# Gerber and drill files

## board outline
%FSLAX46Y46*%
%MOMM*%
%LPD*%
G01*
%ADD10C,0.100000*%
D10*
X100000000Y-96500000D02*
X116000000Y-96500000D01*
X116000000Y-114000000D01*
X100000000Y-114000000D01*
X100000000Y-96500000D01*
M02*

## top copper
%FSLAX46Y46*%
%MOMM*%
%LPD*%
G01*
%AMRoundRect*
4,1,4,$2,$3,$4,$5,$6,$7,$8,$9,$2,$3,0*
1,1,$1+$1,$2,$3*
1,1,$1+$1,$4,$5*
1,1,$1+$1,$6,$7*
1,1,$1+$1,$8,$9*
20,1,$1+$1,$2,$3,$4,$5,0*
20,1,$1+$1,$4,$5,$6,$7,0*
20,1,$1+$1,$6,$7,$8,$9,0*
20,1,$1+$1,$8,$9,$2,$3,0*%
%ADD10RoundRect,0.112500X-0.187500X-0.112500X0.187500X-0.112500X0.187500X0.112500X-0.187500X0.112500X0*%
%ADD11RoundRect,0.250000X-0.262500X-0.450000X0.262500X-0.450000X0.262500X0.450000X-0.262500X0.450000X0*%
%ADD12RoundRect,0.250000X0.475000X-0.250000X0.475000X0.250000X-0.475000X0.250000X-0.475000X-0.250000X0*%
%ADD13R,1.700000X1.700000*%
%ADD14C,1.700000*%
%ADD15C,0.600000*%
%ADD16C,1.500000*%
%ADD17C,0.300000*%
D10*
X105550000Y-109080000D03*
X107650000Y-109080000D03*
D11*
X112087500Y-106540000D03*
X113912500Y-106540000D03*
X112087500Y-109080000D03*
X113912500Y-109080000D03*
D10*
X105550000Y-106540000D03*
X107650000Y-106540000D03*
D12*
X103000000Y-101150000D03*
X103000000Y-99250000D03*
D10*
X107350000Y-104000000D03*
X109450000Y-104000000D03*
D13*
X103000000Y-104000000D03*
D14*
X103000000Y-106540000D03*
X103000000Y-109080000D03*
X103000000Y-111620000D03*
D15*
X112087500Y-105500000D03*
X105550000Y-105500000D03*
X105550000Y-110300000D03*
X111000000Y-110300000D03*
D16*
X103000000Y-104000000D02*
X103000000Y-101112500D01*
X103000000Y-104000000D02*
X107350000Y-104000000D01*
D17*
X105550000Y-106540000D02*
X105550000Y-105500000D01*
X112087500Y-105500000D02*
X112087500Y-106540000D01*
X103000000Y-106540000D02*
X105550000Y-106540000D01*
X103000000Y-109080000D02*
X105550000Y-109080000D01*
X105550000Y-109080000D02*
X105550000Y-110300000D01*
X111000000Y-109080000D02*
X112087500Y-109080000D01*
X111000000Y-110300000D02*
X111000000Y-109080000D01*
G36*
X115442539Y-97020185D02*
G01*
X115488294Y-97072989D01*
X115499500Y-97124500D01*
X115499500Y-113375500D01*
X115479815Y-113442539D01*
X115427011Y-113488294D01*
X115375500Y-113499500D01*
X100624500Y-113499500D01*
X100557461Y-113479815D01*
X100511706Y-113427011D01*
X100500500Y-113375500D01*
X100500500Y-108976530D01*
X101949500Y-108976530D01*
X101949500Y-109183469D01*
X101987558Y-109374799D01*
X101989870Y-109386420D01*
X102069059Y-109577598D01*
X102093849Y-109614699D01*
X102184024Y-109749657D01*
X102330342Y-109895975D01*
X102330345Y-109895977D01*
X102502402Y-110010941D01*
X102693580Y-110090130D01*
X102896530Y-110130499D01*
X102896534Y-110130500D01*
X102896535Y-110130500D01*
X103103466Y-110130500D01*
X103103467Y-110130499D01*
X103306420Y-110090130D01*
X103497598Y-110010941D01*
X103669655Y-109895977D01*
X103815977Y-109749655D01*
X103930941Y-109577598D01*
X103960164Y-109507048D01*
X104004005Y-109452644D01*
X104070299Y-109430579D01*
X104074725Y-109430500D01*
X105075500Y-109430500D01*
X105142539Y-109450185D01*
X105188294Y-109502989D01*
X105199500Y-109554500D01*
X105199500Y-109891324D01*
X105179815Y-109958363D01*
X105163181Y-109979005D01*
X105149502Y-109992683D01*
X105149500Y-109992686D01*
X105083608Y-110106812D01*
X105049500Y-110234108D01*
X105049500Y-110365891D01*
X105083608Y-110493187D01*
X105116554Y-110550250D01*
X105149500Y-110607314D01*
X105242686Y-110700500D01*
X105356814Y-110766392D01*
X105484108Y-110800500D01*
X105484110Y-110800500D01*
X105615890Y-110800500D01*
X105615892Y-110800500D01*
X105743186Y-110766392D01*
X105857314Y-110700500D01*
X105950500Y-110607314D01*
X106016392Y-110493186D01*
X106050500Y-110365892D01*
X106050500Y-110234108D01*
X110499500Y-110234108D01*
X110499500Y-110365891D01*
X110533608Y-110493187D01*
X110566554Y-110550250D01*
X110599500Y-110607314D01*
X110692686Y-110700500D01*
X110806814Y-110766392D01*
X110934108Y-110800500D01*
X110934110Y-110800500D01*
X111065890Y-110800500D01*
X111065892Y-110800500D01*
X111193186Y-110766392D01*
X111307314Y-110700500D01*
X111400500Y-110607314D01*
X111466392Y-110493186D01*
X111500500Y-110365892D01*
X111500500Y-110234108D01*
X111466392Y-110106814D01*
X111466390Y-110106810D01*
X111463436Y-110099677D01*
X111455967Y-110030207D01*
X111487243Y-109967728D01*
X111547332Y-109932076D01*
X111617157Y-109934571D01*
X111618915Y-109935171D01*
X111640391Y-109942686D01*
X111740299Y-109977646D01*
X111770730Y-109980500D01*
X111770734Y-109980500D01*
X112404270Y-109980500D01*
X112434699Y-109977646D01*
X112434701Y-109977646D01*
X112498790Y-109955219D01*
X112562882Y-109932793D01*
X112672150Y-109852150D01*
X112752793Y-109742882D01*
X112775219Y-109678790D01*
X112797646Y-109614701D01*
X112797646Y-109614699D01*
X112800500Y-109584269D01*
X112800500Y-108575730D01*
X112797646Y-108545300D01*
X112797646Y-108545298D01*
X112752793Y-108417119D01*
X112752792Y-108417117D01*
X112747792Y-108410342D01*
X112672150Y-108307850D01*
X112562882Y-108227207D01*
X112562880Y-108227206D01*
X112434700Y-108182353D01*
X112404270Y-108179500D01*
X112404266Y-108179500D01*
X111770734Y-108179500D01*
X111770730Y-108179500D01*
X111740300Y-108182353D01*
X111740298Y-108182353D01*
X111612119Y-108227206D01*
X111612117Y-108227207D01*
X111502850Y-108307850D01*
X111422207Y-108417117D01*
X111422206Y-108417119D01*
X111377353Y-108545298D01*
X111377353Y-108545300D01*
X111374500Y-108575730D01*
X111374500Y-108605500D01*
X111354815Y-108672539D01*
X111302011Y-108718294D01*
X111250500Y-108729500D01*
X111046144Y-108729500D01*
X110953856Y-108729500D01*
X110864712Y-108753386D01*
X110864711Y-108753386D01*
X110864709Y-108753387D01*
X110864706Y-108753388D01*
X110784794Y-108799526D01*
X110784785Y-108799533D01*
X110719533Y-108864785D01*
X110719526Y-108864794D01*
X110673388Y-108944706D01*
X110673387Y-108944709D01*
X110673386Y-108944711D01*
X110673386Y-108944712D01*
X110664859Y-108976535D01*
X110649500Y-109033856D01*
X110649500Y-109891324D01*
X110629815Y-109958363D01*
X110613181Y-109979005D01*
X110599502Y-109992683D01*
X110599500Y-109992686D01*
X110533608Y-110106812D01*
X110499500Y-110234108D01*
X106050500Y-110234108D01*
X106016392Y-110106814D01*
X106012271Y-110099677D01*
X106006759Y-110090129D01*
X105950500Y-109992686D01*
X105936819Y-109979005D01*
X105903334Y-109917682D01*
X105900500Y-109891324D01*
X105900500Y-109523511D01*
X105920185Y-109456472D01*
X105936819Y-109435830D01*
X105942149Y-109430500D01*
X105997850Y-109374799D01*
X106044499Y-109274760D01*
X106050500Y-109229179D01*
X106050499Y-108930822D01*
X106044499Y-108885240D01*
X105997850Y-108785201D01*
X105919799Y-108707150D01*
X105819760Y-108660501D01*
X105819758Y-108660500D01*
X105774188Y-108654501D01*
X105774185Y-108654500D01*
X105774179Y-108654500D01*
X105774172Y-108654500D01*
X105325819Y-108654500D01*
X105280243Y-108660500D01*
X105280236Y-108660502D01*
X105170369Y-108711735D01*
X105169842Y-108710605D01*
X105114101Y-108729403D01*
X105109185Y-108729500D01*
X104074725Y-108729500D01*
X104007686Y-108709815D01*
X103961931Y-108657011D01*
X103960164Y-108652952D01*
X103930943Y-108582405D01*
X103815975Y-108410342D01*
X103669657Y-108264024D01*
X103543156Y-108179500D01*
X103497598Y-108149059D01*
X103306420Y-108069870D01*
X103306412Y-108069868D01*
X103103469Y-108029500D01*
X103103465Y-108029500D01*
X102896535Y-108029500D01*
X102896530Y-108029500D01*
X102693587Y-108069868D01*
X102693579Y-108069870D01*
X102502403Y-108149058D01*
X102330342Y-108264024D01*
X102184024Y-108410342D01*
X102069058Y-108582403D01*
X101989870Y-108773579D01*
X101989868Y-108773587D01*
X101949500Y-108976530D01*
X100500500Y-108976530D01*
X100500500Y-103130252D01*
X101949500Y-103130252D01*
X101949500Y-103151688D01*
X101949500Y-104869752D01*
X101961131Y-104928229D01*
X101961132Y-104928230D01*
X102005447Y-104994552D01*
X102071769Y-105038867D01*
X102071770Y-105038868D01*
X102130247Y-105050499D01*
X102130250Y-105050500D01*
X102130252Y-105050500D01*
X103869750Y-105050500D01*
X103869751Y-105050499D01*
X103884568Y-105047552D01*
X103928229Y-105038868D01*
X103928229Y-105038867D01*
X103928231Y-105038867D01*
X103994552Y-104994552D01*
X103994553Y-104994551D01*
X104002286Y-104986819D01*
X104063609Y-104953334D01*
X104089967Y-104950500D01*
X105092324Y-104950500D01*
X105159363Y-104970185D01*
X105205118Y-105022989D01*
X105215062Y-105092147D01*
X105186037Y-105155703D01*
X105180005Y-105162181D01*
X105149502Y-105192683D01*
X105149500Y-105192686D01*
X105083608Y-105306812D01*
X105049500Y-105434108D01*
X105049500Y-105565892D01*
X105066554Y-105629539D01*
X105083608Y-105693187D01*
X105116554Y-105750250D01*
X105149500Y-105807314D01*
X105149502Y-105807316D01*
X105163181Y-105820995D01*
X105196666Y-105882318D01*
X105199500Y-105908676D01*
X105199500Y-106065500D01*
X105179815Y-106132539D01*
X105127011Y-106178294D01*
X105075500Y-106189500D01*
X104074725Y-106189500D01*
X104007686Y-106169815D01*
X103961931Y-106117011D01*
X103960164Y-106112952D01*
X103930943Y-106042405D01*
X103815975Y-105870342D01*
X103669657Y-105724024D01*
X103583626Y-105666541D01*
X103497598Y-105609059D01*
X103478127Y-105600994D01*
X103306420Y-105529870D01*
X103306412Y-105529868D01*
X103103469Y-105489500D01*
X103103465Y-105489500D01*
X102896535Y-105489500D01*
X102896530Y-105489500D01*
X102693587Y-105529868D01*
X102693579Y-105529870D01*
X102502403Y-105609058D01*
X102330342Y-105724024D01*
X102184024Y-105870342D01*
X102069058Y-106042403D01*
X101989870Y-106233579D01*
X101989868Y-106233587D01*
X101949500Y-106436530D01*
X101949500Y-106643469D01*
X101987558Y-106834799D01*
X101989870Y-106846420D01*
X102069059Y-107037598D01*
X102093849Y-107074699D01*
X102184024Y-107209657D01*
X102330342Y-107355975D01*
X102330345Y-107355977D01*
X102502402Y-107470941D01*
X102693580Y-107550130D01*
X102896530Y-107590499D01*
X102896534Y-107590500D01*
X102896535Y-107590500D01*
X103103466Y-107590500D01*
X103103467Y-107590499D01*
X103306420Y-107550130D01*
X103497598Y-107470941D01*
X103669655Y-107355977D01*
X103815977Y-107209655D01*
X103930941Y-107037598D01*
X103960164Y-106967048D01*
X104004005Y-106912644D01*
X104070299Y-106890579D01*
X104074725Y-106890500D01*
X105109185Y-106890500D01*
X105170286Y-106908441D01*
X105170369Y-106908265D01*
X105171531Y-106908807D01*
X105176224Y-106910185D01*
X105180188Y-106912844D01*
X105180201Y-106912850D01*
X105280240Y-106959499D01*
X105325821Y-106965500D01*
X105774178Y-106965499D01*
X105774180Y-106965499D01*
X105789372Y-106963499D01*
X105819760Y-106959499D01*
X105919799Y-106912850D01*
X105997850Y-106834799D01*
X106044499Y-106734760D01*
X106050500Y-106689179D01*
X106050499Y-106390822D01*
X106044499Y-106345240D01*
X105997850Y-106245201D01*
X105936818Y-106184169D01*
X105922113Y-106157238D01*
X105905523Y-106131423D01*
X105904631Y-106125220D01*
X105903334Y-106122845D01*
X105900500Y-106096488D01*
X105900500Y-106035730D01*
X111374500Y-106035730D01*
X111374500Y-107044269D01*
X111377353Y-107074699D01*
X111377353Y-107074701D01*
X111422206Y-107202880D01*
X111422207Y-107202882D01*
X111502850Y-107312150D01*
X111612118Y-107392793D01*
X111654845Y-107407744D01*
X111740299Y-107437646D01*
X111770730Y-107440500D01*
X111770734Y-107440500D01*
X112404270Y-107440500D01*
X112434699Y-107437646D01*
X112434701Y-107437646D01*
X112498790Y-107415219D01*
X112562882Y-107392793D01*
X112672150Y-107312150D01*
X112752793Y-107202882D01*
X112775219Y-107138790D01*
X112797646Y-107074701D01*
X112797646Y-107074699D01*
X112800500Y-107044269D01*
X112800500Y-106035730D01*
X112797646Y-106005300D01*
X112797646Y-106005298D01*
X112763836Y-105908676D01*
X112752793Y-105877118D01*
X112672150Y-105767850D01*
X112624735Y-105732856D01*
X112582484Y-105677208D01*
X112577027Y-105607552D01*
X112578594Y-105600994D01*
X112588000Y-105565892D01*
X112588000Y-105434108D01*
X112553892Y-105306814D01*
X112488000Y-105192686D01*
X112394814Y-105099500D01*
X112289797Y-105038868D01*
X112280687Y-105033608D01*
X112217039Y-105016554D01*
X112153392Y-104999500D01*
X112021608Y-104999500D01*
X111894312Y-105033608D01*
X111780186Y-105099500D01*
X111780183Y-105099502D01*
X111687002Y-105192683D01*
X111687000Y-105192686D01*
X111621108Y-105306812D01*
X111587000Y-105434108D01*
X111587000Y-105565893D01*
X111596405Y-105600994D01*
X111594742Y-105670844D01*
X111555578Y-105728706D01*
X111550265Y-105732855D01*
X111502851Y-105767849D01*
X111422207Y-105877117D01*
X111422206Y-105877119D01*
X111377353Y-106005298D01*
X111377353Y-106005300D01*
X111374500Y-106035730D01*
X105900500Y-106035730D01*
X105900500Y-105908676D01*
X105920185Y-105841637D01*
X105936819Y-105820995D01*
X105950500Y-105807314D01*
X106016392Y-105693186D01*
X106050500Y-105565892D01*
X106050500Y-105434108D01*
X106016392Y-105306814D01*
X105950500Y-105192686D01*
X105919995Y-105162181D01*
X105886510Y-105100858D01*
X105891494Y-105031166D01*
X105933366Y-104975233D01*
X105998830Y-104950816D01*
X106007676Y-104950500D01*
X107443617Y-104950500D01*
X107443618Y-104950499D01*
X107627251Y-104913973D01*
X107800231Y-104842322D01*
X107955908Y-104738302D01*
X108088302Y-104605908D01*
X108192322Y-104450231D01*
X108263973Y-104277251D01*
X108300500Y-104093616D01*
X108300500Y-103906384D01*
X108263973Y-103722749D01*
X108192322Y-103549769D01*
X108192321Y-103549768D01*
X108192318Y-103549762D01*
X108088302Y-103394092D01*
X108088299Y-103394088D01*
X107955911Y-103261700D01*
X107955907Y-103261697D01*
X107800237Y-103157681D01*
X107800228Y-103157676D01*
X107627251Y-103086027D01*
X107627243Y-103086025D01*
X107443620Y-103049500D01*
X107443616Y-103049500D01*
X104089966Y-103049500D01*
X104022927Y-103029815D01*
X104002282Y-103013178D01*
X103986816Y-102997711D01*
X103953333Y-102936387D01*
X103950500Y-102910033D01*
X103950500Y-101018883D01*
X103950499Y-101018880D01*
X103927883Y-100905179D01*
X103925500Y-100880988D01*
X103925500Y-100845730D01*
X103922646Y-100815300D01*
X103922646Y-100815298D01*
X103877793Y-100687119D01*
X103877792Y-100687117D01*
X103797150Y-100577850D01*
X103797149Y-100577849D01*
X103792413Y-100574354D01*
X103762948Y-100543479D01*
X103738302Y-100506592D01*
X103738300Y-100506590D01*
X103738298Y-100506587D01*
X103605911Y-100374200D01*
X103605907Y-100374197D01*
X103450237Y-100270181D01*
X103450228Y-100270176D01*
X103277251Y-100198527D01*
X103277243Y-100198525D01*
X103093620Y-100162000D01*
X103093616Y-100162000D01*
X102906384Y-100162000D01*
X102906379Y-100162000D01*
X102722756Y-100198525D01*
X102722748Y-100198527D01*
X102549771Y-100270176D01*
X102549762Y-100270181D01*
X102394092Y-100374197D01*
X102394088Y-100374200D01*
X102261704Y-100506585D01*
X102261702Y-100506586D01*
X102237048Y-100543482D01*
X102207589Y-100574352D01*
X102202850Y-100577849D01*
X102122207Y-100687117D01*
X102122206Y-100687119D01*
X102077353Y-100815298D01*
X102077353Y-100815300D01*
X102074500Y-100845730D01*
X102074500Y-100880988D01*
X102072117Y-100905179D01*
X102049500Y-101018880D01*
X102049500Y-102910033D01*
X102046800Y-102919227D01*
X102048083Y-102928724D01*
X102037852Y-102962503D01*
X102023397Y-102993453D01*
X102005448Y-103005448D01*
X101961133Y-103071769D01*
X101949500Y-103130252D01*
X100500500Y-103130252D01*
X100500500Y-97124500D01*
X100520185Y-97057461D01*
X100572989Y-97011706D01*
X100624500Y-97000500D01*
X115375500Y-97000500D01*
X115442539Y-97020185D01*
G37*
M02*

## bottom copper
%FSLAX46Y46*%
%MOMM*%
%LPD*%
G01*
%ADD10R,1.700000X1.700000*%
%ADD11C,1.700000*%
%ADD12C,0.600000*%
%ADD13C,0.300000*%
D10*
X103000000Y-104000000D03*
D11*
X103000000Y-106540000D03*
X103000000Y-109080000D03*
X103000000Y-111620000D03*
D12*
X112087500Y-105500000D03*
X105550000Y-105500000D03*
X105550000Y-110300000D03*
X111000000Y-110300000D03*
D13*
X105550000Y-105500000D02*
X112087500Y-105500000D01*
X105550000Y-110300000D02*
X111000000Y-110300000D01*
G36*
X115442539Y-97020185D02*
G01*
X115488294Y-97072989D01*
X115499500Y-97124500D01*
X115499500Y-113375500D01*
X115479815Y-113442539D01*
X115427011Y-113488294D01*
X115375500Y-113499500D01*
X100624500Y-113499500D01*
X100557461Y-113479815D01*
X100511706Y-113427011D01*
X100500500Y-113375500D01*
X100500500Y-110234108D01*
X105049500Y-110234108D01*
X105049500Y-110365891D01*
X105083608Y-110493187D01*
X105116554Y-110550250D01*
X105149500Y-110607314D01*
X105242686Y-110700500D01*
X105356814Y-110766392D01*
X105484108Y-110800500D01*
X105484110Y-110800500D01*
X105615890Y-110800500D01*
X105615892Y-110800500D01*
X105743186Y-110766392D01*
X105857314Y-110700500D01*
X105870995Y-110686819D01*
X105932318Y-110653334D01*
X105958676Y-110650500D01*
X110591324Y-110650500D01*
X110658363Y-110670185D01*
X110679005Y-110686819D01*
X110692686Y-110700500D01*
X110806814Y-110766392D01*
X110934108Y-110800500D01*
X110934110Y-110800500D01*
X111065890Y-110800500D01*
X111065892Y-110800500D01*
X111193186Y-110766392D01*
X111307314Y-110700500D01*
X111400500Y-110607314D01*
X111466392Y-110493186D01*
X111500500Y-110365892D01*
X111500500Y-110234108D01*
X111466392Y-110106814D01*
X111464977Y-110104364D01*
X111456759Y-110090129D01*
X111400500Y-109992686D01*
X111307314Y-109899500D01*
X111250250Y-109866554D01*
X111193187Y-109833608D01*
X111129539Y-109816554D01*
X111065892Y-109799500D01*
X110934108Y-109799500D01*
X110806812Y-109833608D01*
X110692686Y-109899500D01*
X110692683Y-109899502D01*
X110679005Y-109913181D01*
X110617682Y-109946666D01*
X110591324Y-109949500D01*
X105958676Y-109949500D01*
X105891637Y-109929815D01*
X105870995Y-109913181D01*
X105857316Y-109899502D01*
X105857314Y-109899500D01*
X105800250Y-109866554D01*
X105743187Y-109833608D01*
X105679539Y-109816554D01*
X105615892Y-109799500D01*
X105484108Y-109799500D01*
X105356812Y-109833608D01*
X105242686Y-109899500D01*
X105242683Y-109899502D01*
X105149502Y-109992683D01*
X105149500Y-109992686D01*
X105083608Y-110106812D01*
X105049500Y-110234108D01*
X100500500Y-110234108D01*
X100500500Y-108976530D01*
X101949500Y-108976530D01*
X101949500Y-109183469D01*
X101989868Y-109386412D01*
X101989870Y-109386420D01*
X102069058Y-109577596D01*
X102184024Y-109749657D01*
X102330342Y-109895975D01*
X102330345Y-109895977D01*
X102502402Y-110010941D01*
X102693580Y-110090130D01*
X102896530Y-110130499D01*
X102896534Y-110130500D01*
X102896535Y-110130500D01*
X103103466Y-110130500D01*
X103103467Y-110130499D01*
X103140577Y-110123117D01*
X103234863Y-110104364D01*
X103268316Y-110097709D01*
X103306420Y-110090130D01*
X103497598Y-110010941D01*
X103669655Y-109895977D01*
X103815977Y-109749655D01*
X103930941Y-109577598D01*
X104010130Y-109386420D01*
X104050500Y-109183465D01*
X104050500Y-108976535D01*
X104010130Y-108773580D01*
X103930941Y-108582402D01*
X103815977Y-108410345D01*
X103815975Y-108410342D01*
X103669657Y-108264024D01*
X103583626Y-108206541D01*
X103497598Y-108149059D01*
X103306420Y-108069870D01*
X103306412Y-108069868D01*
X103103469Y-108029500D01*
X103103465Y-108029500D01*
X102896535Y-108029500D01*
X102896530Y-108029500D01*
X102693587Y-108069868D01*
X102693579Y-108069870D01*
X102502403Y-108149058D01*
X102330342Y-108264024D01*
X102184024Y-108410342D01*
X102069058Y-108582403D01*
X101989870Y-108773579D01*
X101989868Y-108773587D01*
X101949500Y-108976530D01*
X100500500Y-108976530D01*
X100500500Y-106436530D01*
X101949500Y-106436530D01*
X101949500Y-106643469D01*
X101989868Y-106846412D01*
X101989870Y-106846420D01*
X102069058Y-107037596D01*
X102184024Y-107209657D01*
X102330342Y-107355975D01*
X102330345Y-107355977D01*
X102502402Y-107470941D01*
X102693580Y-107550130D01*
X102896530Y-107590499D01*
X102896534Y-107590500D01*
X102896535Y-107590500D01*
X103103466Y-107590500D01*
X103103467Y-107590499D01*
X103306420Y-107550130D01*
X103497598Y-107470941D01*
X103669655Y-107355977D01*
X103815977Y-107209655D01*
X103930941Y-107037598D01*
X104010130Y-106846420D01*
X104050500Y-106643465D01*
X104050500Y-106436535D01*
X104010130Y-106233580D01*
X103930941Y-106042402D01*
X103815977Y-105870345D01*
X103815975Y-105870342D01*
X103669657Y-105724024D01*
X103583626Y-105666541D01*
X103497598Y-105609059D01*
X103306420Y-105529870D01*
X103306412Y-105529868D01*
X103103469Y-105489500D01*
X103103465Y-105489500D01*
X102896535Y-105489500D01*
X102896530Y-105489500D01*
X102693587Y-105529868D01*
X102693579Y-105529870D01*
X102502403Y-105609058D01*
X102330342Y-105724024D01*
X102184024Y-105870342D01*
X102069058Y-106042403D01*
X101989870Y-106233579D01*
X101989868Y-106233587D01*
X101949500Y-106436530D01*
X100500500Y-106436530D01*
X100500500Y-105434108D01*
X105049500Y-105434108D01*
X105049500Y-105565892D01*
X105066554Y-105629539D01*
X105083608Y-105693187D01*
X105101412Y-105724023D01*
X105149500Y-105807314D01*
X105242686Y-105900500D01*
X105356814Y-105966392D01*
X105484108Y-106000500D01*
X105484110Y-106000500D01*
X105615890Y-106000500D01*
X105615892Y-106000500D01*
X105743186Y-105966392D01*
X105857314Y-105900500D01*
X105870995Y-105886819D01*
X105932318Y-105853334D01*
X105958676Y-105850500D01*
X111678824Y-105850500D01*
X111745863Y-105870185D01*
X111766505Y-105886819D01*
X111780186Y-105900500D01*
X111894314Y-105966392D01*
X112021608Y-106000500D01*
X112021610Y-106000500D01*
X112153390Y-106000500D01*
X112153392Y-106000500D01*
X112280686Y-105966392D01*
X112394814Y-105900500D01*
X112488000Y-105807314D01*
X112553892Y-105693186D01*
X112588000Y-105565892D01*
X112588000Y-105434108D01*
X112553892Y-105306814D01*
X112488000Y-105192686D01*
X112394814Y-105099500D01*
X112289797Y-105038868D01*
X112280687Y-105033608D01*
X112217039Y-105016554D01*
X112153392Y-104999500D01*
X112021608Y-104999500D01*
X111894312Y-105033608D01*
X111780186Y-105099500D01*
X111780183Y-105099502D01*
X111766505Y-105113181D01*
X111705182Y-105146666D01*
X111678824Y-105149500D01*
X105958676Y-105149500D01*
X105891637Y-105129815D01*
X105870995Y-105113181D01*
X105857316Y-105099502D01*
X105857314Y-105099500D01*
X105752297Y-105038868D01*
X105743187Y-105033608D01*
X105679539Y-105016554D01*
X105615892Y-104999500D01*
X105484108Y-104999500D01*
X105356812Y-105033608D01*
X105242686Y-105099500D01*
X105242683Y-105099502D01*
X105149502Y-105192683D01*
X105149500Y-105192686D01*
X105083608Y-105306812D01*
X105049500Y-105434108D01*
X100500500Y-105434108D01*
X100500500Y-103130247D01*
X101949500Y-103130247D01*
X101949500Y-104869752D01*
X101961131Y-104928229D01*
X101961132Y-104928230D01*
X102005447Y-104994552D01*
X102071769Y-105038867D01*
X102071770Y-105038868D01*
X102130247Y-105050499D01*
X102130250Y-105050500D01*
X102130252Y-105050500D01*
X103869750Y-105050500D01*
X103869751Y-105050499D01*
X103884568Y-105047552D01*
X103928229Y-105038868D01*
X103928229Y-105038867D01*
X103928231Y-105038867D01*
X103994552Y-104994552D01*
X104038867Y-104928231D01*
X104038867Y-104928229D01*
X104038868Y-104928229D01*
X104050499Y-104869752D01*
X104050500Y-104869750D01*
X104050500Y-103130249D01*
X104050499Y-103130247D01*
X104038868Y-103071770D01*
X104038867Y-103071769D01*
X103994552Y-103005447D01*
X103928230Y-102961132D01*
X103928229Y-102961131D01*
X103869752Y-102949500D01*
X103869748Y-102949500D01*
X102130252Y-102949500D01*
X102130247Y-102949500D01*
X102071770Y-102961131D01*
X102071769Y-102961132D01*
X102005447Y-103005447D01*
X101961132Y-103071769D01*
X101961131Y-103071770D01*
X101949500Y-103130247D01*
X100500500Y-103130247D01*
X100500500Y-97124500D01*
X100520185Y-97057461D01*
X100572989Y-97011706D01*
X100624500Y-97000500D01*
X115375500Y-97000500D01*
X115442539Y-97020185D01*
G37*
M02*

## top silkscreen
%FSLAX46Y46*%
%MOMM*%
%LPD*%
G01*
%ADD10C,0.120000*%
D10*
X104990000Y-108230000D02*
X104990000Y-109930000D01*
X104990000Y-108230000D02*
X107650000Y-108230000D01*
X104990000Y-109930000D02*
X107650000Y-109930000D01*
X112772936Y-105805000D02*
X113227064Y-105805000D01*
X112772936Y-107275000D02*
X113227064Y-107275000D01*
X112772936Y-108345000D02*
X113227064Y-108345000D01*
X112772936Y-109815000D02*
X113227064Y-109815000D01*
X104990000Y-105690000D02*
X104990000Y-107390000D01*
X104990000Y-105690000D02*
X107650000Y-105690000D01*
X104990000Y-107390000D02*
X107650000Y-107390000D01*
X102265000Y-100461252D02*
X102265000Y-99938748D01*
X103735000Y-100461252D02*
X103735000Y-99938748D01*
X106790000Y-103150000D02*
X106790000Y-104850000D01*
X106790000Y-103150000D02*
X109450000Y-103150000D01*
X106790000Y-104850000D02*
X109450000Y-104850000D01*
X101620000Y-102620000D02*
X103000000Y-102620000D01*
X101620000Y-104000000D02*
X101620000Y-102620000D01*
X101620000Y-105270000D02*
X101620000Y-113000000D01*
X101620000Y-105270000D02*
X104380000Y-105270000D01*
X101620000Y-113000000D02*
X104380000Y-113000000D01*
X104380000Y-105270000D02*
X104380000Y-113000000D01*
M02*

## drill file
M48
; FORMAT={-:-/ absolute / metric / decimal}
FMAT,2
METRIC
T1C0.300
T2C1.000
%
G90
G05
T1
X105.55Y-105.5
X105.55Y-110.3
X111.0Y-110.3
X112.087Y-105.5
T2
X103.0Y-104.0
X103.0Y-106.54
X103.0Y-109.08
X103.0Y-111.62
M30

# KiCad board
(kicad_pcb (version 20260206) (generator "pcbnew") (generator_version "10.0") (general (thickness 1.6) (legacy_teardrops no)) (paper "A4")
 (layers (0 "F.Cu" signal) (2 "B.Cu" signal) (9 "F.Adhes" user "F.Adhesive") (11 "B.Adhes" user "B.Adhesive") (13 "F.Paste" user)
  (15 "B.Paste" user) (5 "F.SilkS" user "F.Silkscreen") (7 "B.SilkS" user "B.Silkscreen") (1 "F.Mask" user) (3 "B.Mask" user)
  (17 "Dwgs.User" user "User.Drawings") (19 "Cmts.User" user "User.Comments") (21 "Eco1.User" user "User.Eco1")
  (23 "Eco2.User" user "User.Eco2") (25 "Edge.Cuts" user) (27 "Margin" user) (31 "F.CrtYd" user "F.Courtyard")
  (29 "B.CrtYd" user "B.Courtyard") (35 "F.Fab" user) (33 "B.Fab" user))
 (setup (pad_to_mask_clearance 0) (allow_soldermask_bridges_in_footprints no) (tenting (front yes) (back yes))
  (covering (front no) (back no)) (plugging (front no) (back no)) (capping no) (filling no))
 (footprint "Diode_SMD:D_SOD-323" (layer "F.Cu") (at 106.6 109.08)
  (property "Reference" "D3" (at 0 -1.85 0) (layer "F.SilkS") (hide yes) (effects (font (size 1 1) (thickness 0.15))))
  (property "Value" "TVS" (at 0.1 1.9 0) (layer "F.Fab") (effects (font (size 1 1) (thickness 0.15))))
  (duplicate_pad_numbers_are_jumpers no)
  (fp_line (start -1.61 -0.85) (end -1.61 0.85) (stroke (width 0.12) (type solid)) (layer "F.SilkS"))
  (fp_line (start -1.61 -0.85) (end 1.05 -0.85) (stroke (width 0.12) (type solid)) (layer "F.SilkS"))
  (fp_line (start -1.61 0.85) (end 1.05 0.85) (stroke (width 0.12) (type solid)) (layer "F.SilkS"))
  (pad "1" smd roundrect (at -1.05 0) (size 0.6 0.45) (layers "F.Cu" "F.Mask" "F.Paste") (roundrect_rratio 0.25) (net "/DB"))
  (pad "2" smd roundrect (at 1.05 0) (size 0.6 0.45) (layers "F.Cu" "F.Mask" "F.Paste") (roundrect_rratio 0.25) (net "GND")))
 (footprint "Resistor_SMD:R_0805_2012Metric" (layer "F.Cu") (at 113 106.54)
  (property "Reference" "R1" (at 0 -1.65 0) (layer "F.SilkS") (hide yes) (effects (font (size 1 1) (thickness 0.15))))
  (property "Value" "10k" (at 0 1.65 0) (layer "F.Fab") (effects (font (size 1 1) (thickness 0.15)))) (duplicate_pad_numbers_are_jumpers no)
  (fp_line (start -0.227064 -0.735) (end 0.227064 -0.735) (stroke (width 0.12) (type solid)) (layer "F.SilkS"))
  (fp_line (start -0.227064 0.735) (end 0.227064 0.735) (stroke (width 0.12) (type solid)) (layer "F.SilkS"))
  (pad "1" smd roundrect (at -0.9125 0) (size 1.025 1.4) (layers "F.Cu" "F.Mask" "F.Paste") (roundrect_rratio 0.243902) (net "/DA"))
  (pad "2" smd roundrect (at 0.9125 0) (size 1.025 1.4) (layers "F.Cu" "F.Mask" "F.Paste") (roundrect_rratio 0.243902) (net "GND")))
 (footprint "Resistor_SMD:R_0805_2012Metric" (layer "F.Cu") (at 113 109.08)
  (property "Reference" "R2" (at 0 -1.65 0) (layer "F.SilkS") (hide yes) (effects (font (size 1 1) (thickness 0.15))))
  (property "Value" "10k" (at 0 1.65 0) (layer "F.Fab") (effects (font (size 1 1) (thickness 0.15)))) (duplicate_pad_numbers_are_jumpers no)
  (fp_line (start -0.227064 -0.735) (end 0.227064 -0.735) (stroke (width 0.12) (type solid)) (layer "F.SilkS"))
  (fp_line (start -0.227064 0.735) (end 0.227064 0.735) (stroke (width 0.12) (type solid)) (layer "F.SilkS"))
  (pad "1" smd roundrect (at -0.9125 0) (size 1.025 1.4) (layers "F.Cu" "F.Mask" "F.Paste") (roundrect_rratio 0.243902) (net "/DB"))
  (pad "2" smd roundrect (at 0.9125 0) (size 1.025 1.4) (layers "F.Cu" "F.Mask" "F.Paste") (roundrect_rratio 0.243902) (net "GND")))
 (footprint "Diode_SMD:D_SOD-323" (layer "F.Cu") (at 106.6 106.54)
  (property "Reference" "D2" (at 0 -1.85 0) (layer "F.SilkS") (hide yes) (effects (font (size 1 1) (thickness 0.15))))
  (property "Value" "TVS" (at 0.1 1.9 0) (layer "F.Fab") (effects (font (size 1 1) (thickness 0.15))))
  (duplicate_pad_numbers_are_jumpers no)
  (fp_line (start -1.61 -0.85) (end -1.61 0.85) (stroke (width 0.12) (type solid)) (layer "F.SilkS"))
  (fp_line (start -1.61 -0.85) (end 1.05 -0.85) (stroke (width 0.12) (type solid)) (layer "F.SilkS"))
  (fp_line (start -1.61 0.85) (end 1.05 0.85) (stroke (width 0.12) (type solid)) (layer "F.SilkS"))
  (pad "1" smd roundrect (at -1.05 0) (size 0.6 0.45) (layers "F.Cu" "F.Mask" "F.Paste") (roundrect_rratio 0.25) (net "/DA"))
  (pad "2" smd roundrect (at 1.05 0) (size 0.6 0.45) (layers "F.Cu" "F.Mask" "F.Paste") (roundrect_rratio 0.25) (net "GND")))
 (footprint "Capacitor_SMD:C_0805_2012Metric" (layer "F.Cu") (at 103 100.2 90)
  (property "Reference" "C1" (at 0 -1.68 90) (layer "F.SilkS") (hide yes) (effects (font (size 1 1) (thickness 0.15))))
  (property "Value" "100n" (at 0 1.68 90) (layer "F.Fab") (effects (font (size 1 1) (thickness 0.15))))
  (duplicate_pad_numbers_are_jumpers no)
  (fp_line (start -0.261252 -0.735) (end 0.261252 -0.735) (stroke (width 0.12) (type solid)) (layer "F.SilkS"))
  (fp_line (start -0.261252 0.735) (end 0.261252 0.735) (stroke (width 0.12) (type solid)) (layer "F.SilkS"))
  (pad "1" smd roundrect (at -0.95 0 90) (size 1 1.45) (layers "F.Cu" "F.Mask" "F.Paste") (roundrect_rratio 0.25) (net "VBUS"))
  (pad "2" smd roundrect (at 0.95 0 90) (size 1 1.45) (layers "F.Cu" "F.Mask" "F.Paste") (roundrect_rratio 0.25) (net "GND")))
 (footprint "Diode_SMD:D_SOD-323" (layer "F.Cu") (at 108.4 104)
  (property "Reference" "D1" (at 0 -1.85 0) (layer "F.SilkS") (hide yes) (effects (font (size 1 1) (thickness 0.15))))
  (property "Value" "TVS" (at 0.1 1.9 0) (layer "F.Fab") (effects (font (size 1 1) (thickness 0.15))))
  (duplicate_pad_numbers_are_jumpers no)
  (fp_line (start -1.61 -0.85) (end -1.61 0.85) (stroke (width 0.12) (type solid)) (layer "F.SilkS"))
  (fp_line (start -1.61 -0.85) (end 1.05 -0.85) (stroke (width 0.12) (type solid)) (layer "F.SilkS"))
  (fp_line (start -1.61 0.85) (end 1.05 0.85) (stroke (width 0.12) (type solid)) (layer "F.SilkS"))
  (pad "1" smd roundrect (at -1.05 0) (size 0.6 0.45) (layers "F.Cu" "F.Mask" "F.Paste") (roundrect_rratio 0.25) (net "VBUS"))
  (pad "2" smd roundrect (at 1.05 0) (size 0.6 0.45) (layers "F.Cu" "F.Mask" "F.Paste") (roundrect_rratio 0.25) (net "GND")))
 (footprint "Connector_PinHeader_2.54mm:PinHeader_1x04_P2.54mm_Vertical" (layer "F.Cu") (at 103 104)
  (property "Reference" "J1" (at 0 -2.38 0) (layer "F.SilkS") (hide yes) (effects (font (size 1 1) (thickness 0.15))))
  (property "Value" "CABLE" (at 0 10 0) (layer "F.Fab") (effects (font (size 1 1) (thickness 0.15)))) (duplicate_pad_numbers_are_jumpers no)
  (fp_line (start -1.38 -1.38) (end 0 -1.38) (stroke (width 0.12) (type solid)) (layer "F.SilkS"))
  (fp_line (start -1.38 0) (end -1.38 -1.38) (stroke (width 0.12) (type solid)) (layer "F.SilkS"))
  (fp_line (start -1.38 1.27) (end -1.38 9) (stroke (width 0.12) (type solid)) (layer "F.SilkS"))
  (fp_line (start -1.38 1.27) (end 1.38 1.27) (stroke (width 0.12) (type solid)) (layer "F.SilkS"))
  (fp_line (start -1.38 9) (end 1.38 9) (stroke (width 0.12) (type solid)) (layer "F.SilkS"))
  (fp_line (start 1.38 1.27) (end 1.38 9) (stroke (width 0.12) (type solid)) (layer "F.SilkS"))
  (pad "1" thru_hole rect (at 0 0) (size 1.7 1.7) (drill 1) (layers "*.Cu" "*.Mask") (remove_unused_layers no) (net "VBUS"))
  (pad "2" thru_hole circle (at 0 2.54) (size 1.7 1.7) (drill 1) (layers "*.Cu" "*.Mask") (remove_unused_layers no) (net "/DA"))
  (pad "3" thru_hole circle (at 0 5.08) (size 1.7 1.7) (drill 1) (layers "*.Cu" "*.Mask") (remove_unused_layers no) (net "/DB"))
  (pad "4" thru_hole circle (at 0 7.62) (size 1.7 1.7) (drill 1) (layers "*.Cu" "*.Mask") (remove_unused_layers no) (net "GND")))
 (gr_rect (start 100 96.5) (end 116 114) (stroke (width 0.1) (type default)) (fill no) (layer "Edge.Cuts"))
 (segment (start 103 104) (end 103 101.1125) (width 1.5) (layer "F.Cu") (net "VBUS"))
 (segment (start 103 104) (end 107.35 104) (width 1.5) (layer "F.Cu") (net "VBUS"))
 (segment (start 105.55 106.54) (end 105.55 105.5) (width 0.3) (layer "F.Cu") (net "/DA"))
 (segment (start 112.0875 105.5) (end 112.0875 106.54) (width 0.3) (layer "F.Cu") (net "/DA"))
 (segment (start 103 106.54) (end 105.55 106.54) (width 0.3) (layer "F.Cu") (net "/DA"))
 (via (at 112.0875 105.5) (size 0.6) (drill 0.3) (layers "F.Cu" "B.Cu") (capping no) (covering (front no) (back no))
  (plugging (front no) (back no)) (filling no) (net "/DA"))
 (via (at 105.55 105.5) (size 0.6) (drill 0.3) (layers "F.Cu" "B.Cu") (capping no) (covering (front no) (back no))
  (plugging (front no) (back no)) (filling no) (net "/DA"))
 (segment (start 105.55 105.5) (end 112.0875 105.5) (width 0.3) (layer "B.Cu") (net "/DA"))
 (segment (start 103 109.08) (end 105.55 109.08) (width 0.3) (layer "F.Cu") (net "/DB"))
 (segment (start 105.55 109.08) (end 105.55 110.3) (width 0.3) (layer "F.Cu") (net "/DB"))
 (segment (start 111 109.08) (end 112.0875 109.08) (width 0.3) (layer "F.Cu") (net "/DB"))
 (segment (start 111 110.3) (end 111 109.08) (width 0.3) (layer "F.Cu") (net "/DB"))
 (via (at 105.55 110.3) (size 0.6) (drill 0.3) (layers "F.Cu" "B.Cu") (capping no) (covering (front no) (back no))
  (plugging (front no) (back no)) (filling no) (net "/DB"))
 (via (at 111 110.3) (size 0.6) (drill 0.3) (layers "F.Cu" "B.Cu") (capping no) (covering (front no) (back no))
  (plugging (front no) (back no)) (filling no) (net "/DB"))
 (segment (start 105.55 110.3) (end 111 110.3) (width 0.3) (layer "B.Cu") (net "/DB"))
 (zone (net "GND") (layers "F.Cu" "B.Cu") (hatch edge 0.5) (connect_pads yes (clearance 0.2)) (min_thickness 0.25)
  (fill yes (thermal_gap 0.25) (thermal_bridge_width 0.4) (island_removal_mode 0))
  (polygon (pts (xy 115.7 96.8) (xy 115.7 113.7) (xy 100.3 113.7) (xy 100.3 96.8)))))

